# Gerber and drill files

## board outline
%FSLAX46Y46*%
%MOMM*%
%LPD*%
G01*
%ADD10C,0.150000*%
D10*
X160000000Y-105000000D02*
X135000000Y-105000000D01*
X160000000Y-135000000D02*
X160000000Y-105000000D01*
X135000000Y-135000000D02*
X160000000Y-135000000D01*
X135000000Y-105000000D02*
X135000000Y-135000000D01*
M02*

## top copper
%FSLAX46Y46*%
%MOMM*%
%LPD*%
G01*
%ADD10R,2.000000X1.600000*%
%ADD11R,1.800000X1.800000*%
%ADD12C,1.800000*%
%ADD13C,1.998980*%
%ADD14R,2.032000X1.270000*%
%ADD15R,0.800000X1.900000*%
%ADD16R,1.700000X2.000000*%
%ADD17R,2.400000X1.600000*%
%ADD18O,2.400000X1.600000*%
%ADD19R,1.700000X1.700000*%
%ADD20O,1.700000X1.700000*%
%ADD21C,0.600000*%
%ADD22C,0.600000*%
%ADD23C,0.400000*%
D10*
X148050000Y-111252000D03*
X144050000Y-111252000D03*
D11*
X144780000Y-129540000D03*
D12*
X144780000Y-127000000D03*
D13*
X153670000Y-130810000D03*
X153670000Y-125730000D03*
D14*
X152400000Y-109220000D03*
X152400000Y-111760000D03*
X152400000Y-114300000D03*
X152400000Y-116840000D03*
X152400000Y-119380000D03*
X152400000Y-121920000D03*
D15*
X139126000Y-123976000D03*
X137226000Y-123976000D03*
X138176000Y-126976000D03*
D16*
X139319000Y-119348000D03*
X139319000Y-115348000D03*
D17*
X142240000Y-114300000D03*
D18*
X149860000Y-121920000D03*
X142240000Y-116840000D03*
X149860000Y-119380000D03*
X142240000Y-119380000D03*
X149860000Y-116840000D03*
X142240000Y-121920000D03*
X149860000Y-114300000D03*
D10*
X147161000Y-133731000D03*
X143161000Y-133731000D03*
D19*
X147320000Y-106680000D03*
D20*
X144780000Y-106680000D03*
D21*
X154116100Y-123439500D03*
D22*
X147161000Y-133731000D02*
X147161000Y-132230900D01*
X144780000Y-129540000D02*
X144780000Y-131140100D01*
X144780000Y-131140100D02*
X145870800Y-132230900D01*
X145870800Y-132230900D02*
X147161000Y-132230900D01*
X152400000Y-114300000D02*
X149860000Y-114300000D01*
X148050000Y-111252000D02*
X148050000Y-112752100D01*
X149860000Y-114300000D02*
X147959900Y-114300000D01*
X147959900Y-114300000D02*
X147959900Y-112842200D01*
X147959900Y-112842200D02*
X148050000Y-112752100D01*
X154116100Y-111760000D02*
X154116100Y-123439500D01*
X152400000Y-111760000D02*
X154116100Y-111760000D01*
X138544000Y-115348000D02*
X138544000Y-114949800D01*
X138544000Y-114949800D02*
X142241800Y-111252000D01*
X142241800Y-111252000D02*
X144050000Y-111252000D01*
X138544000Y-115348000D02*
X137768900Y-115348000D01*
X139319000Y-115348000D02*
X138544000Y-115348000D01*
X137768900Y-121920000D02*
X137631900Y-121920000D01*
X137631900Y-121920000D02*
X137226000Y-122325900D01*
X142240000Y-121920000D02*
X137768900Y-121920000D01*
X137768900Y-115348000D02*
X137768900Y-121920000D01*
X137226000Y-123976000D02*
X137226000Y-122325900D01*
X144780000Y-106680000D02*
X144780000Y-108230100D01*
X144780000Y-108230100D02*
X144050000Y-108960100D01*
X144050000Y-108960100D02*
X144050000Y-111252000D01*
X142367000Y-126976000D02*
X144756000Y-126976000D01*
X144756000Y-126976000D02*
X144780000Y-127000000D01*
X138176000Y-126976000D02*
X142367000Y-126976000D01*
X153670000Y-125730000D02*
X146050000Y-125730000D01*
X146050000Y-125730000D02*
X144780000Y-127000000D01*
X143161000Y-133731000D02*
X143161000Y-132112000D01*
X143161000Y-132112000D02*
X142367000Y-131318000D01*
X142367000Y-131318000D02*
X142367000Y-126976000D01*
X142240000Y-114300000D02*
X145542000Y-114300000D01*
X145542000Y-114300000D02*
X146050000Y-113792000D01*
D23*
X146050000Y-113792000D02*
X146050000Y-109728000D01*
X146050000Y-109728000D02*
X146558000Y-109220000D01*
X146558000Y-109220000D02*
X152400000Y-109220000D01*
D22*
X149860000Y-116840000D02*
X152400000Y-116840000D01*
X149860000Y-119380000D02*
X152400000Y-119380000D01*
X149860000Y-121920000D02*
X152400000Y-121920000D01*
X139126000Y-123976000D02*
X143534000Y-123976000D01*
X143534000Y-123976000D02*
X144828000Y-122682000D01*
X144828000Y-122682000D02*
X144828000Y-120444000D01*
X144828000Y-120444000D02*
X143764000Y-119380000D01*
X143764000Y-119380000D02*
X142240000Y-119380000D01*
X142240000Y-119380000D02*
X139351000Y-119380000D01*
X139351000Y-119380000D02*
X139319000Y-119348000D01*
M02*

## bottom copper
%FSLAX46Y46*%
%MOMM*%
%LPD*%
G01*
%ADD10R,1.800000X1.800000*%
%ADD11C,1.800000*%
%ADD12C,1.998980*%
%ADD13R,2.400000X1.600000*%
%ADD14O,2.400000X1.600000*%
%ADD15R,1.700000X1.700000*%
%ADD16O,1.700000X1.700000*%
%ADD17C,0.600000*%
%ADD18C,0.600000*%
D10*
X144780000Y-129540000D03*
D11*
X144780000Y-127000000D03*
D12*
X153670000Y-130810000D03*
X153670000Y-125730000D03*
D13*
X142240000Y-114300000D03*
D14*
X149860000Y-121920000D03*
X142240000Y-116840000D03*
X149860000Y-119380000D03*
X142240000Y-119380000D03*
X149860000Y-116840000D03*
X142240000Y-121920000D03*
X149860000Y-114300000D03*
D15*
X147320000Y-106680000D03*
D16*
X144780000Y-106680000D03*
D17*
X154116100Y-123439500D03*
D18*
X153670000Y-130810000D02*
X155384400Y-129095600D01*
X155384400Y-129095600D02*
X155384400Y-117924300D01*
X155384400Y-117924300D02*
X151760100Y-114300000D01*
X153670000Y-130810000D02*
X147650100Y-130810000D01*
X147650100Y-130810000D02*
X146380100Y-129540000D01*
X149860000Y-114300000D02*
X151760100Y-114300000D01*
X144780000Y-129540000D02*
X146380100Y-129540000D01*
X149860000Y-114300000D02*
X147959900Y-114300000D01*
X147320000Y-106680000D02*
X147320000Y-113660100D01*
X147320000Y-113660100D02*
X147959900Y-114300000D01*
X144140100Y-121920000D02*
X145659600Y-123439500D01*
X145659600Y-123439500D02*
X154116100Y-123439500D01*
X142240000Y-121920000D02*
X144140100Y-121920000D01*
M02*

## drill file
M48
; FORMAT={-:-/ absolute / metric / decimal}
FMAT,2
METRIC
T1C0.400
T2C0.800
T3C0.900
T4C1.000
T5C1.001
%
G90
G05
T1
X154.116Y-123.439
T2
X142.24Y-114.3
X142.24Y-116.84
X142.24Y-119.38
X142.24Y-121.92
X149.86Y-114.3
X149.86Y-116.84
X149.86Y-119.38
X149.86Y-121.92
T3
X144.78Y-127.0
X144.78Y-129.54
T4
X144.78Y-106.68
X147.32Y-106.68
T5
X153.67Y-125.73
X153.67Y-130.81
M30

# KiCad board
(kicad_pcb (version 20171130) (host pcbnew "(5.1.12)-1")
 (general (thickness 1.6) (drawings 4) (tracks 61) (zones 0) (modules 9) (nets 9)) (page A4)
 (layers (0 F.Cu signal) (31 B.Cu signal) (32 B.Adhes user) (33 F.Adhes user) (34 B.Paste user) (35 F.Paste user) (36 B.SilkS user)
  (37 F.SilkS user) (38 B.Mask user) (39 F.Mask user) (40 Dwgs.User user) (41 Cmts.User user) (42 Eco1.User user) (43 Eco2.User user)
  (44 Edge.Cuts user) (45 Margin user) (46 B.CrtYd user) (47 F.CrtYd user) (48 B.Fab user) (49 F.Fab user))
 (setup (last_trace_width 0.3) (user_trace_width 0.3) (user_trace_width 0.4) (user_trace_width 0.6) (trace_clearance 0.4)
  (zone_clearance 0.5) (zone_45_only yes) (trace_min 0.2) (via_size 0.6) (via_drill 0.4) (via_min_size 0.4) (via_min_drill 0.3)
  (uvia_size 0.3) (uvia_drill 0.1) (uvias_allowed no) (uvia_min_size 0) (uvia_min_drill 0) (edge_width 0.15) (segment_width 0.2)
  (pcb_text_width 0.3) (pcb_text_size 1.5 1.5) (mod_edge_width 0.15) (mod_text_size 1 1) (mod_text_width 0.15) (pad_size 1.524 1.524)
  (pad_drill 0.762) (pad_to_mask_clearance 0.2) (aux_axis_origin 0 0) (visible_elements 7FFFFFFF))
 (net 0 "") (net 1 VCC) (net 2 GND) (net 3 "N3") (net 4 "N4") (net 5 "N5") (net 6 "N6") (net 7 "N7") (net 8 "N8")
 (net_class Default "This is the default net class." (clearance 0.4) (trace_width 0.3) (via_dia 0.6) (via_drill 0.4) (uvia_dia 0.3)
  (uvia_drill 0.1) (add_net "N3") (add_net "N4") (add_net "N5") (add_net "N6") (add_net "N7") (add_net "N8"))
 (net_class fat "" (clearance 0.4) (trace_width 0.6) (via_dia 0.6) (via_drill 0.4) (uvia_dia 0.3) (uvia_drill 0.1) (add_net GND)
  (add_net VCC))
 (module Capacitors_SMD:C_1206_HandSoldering (layer F.Cu) (at 146.05 111.252 180)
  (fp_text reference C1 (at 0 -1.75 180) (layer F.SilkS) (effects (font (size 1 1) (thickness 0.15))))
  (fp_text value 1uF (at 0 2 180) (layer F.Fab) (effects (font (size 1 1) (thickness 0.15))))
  (pad 1 smd rect (at -2 0 180) (size 2 1.6) (layers F.Cu F.Paste F.Mask) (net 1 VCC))
  (pad 2 smd rect (at 2 0 180) (size 2 1.6) (layers F.Cu F.Paste F.Mask) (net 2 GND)))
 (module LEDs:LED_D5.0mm (layer F.Cu) (at 144.78 129.54 90)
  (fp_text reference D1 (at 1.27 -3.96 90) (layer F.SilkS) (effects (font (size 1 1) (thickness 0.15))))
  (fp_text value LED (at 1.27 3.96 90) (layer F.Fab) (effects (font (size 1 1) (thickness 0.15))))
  (pad 1 thru_hole rect (at 0 0 90) (size 1.8 1.8) (drill 0.9) (layers *.Cu *.Mask) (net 1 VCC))
  (pad 2 thru_hole circle (at 2.54 0 90) (size 1.8 1.8) (drill 0.9) (layers *.Cu *.Mask) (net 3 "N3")))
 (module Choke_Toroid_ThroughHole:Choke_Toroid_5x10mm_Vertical (layer F.Cu) (at 148.59 130.81)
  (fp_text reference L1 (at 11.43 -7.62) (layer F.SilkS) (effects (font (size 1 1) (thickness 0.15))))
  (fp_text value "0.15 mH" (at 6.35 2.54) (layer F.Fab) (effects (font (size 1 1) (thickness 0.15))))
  (pad 1 thru_hole circle (at 5.08 0) (size 1.99898 1.99898) (drill 1.00076) (layers *.Cu *.Mask) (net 1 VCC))
  (pad 2 thru_hole circle (at 5.08 -5.08) (size 1.99898 1.99898) (drill 1.00076) (layers *.Cu *.Mask) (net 3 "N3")))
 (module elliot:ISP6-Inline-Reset (layer F.Cu) (at 152.4 116.84 270)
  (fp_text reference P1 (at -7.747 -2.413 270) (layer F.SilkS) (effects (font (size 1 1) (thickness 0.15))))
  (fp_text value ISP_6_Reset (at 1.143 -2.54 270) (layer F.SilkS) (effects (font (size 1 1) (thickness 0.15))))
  (pad 1 smd rect (at -7.62 0 270) (size 1.27 2.032) (layers F.Cu F.Paste F.Mask) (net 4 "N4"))
  (pad 2 smd rect (at -5.08 0 270) (size 1.27 2.032) (layers F.Cu F.Paste F.Mask) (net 2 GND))
  (pad 3 smd rect (at -2.54 0 270) (size 1.27 2.032) (layers F.Cu F.Paste F.Mask) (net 1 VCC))
  (pad 4 smd rect (at 0 0 270) (size 1.27 2.032) (layers F.Cu F.Paste F.Mask) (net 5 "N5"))
  (pad 5 smd rect (at 2.54 0 270) (size 1.27 2.032) (layers F.Cu F.Paste F.Mask) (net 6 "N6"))
  (pad 6 smd rect (at 5.08 0 270) (size 1.27 2.032) (layers F.Cu F.Paste F.Mask) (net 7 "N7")))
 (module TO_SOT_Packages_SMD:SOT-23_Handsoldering (layer F.Cu) (at 138.176 125.476 270)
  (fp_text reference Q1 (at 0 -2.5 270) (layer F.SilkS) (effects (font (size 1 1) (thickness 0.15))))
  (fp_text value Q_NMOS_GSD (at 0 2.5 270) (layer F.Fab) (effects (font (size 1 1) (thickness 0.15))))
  (pad 1 smd rect (at -1.5 -0.95 270) (size 1.9 0.8) (layers F.Cu F.Paste F.Mask) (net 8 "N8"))
  (pad 2 smd rect (at -1.5 0.95 270) (size 1.9 0.8) (layers F.Cu F.Paste F.Mask) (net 2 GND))
  (pad 3 smd rect (at 1.5 0 270) (size 1.9 0.8) (layers F.Cu F.Paste F.Mask) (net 3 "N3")))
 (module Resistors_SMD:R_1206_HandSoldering (layer F.Cu) (at 139.319 117.348 90)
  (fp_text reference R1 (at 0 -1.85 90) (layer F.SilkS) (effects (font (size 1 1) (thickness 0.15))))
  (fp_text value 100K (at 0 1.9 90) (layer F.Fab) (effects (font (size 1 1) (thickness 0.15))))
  (pad 1 smd rect (at -2 0 90) (size 2 1.7) (layers F.Cu F.Paste F.Mask) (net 8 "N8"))
  (pad 2 smd rect (at 2 0 90) (size 2 1.7) (layers F.Cu F.Paste F.Mask) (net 2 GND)))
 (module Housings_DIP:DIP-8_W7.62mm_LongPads (layer F.Cu) (at 142.24 114.3)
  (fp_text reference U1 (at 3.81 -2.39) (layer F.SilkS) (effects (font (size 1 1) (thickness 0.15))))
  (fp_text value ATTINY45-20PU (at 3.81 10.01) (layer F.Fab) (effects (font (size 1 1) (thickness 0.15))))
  (pad 1 thru_hole rect (at 0 0) (size 2.4 1.6) (drill 0.8) (layers *.Cu *.Mask) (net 4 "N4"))
  (pad 5 thru_hole oval (at 7.62 7.62) (size 2.4 1.6) (drill 0.8) (layers *.Cu *.Mask) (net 7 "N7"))
  (pad 2 thru_hole oval (at 0 2.54) (size 2.4 1.6) (drill 0.8) (layers *.Cu *.Mask))
  (pad 6 thru_hole oval (at 7.62 5.08) (size 2.4 1.6) (drill 0.8) (layers *.Cu *.Mask) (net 6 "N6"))
  (pad 3 thru_hole oval (at 0 5.08) (size 2.4 1.6) (drill 0.8) (layers *.Cu *.Mask) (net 8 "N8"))
  (pad 7 thru_hole oval (at 7.62 2.54) (size 2.4 1.6) (drill 0.8) (layers *.Cu *.Mask) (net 5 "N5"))
  (pad 4 thru_hole oval (at 0 7.62) (size 2.4 1.6) (drill 0.8) (layers *.Cu *.Mask) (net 2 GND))
  (pad 8 thru_hole oval (at 7.62 0) (size 2.4 1.6) (drill 0.8) (layers *.Cu *.Mask) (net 1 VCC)))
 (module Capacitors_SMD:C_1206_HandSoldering (layer F.Cu) (at 145.161 133.731 180)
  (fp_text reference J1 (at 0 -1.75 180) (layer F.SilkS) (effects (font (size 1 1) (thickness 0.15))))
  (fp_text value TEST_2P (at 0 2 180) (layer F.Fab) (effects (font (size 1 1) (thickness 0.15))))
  (pad 1 smd rect (at -2 0 180) (size 2 1.6) (layers F.Cu F.Paste F.Mask) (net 1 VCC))
  (pad 2 smd rect (at 2 0 180) (size 2 1.6) (layers F.Cu F.Paste F.Mask) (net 3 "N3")))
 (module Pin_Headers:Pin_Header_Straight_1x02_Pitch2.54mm (layer F.Cu) (at 147.32 106.68 270)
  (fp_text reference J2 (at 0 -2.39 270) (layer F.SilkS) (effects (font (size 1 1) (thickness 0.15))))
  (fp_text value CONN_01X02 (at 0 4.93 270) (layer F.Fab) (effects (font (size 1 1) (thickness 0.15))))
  (pad 1 thru_hole rect (at 0 0 270) (size 1.7 1.7) (drill 1) (layers *.Cu *.Mask) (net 1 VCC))
  (pad 2 thru_hole oval (at 0 2.54 270) (size 1.7 1.7) (drill 1) (layers *.Cu *.Mask) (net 2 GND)))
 (gr_line (start 160 105) (end 135 105) (angle 90) (layer Edge.Cuts) (width 0.15))
 (gr_line (start 160 135) (end 160 105) (angle 90) (layer Edge.Cuts) (width 0.15))
 (gr_line (start 135 135) (end 160 135) (angle 90) (layer Edge.Cuts) (width 0.15))
 (gr_line (start 135 105) (end 135 135) (angle 90) (layer Edge.Cuts) (width 0.15))
 (segment (start 153.67 130.81) (end 155.3844 129.0956) (width 0.6) (layer B.Cu) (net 1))
 (segment (start 155.3844 129.0956) (end 155.3844 117.9243) (width 0.6) (layer B.Cu) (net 1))
 (segment (start 155.3844 117.9243) (end 151.7601 114.3) (width 0.6) (layer B.Cu) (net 1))
 (segment (start 153.67 130.81) (end 147.6501 130.81) (width 0.6) (layer B.Cu) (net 1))
 (segment (start 147.6501 130.81) (end 146.3801 129.54) (width 0.6) (layer B.Cu) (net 1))
 (segment (start 149.86 114.3) (end 151.7601 114.3) (width 0.6) (layer B.Cu) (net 1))
 (segment (start 147.161 133.731) (end 147.161 132.2309) (width 0.6) (layer F.Cu) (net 1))
 (segment (start 144.78 129.54) (end 144.78 131.1401) (width 0.6) (layer F.Cu) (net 1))
 (segment (start 144.78 131.1401) (end 145.8708 132.2309) (width 0.6) (layer F.Cu) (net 1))
 (segment (start 145.8708 132.2309) (end 147.161 132.2309) (width 0.6) (layer F.Cu) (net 1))
 (segment (start 144.78 129.54) (end 146.3801 129.54) (width 0.6) (layer B.Cu) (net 1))
 (segment (start 152.4 114.3) (end 149.86 114.3) (width 0.6) (layer F.Cu) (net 1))
 (segment (start 148.05 111.252) (end 148.05 112.7521) (width 0.6) (layer F.Cu) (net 1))
 (segment (start 149.86 114.3) (end 147.9599 114.3) (width 0.6) (layer F.Cu) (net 1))
 (segment (start 147.9599 114.3) (end 147.9599 112.8422) (width 0.6) (layer F.Cu) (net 1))
 (segment (start 147.9599 112.8422) (end 148.05 112.7521) (width 0.6) (layer F.Cu) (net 1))
 (segment (start 149.86 114.3) (end 147.9599 114.3) (width 0.6) (layer B.Cu) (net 1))
 (segment (start 147.32 106.68) (end 147.32 113.6601) (width 0.6) (layer B.Cu) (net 1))
 (segment (start 147.32 113.6601) (end 147.9599 114.3) (width 0.6) (layer B.Cu) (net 1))
 (segment (start 154.1161 111.76) (end 154.1161 123.4395) (width 0.6) (layer F.Cu) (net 2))
 (segment (start 144.1401 121.92) (end 145.6596 123.4395) (width 0.6) (layer B.Cu) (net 2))
 (segment (start 145.6596 123.4395) (end 154.1161 123.4395) (width 0.6) (layer B.Cu) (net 2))
 (segment (start 142.24 121.92) (end 144.1401 121.92) (width 0.6) (layer B.Cu) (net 2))
 (segment (start 152.4 111.76) (end 154.1161 111.76) (width 0.6) (layer F.Cu) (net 2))
 (segment (start 138.544 115.348) (end 138.544 114.9498) (width 0.6) (layer F.Cu) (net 2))
 (segment (start 138.544 114.9498) (end 142.2418 111.252) (width 0.6) (layer F.Cu) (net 2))
 (segment (start 142.2418 111.252) (end 144.05 111.252) (width 0.6) (layer F.Cu) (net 2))
 (segment (start 138.544 115.348) (end 137.7689 115.348) (width 0.6) (layer F.Cu) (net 2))
 (segment (start 139.319 115.348) (end 138.544 115.348) (width 0.6) (layer F.Cu) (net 2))
 (segment (start 137.7689 121.92) (end 137.6319 121.92) (width 0.6) (layer F.Cu) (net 2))
 (segment (start 137.6319 121.92) (end 137.226 122.3259) (width 0.6) (layer F.Cu) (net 2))
 (segment (start 142.24 121.92) (end 137.7689 121.92) (width 0.6) (layer F.Cu) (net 2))
 (segment (start 137.7689 115.348) (end 137.7689 121.92) (width 0.6) (layer F.Cu) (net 2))
 (segment (start 137.226 123.976) (end 137.226 122.3259) (width 0.6) (layer F.Cu) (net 2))
 (segment (start 144.78 106.68) (end 144.78 108.2301) (width 0.6) (layer F.Cu) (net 2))
 (segment (start 144.78 108.2301) (end 144.05 108.9601) (width 0.6) (layer F.Cu) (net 2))
 (segment (start 144.05 108.9601) (end 144.05 111.252) (width 0.6) (layer F.Cu) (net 2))
 (via (at 154.1161 123.4395) (size 0.6) (layers F.Cu B.Cu) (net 2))
 (segment (start 142.367 126.976) (end 144.756 126.976) (width 0.6) (layer F.Cu) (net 3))
 (segment (start 144.756 126.976) (end 144.78 127) (width 0.6) (layer F.Cu) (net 3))
 (segment (start 138.176 126.976) (end 142.367 126.976) (width 0.6) (layer F.Cu) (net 3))
 (segment (start 153.67 125.73) (end 146.05 125.73) (width 0.6) (layer F.Cu) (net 3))
 (segment (start 146.05 125.73) (end 144.78 127) (width 0.6) (layer F.Cu) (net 3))
 (segment (start 143.161 133.731) (end 143.161 132.112) (width 0.6) (layer F.Cu) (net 3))
 (segment (start 143.161 132.112) (end 142.367 131.318) (width 0.6) (layer F.Cu) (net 3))
 (segment (start 142.367 131.318) (end 142.367 126.976) (width 0.6) (layer F.Cu) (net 3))
 (segment (start 142.24 114.3) (end 145.542 114.3) (width 0.6) (layer F.Cu) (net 4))
 (segment (start 145.542 114.3) (end 146.05 113.792) (width 0.6) (layer F.Cu) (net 4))
 (segment (start 146.05 113.792) (end 146.05 109.728) (width 0.4) (layer F.Cu) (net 4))
 (segment (start 146.05 109.728) (end 146.558 109.22) (width 0.4) (layer F.Cu) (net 4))
 (segment (start 146.558 109.22) (end 152.4 109.22) (width 0.4) (layer F.Cu) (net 4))
 (segment (start 149.86 116.84) (end 152.4 116.84) (width 0.6) (layer F.Cu) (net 5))
 (segment (start 149.86 119.38) (end 152.4 119.38) (width 0.6) (layer F.Cu) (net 6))
 (segment (start 149.86 121.92) (end 152.4 121.92) (width 0.6) (layer F.Cu) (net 7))
 (segment (start 139.126 123.976) (end 143.534 123.976) (width 0.6) (layer F.Cu) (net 8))
 (segment (start 143.534 123.976) (end 144.828 122.682) (width 0.6) (layer F.Cu) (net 8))
 (segment (start 144.828 122.682) (end 144.828 120.444) (width 0.6) (layer F.Cu) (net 8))
 (segment (start 144.828 120.444) (end 143.764 119.38) (width 0.6) (layer F.Cu) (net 8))
 (segment (start 143.764 119.38) (end 142.24 119.38) (width 0.6) (layer F.Cu) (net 8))
 (segment (start 142.24 119.38) (end 139.351 119.38) (width 0.6) (layer F.Cu) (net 8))
 (segment (start 139.351 119.38) (end 139.319 119.348) (width 0.6) (layer F.Cu) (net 8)))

